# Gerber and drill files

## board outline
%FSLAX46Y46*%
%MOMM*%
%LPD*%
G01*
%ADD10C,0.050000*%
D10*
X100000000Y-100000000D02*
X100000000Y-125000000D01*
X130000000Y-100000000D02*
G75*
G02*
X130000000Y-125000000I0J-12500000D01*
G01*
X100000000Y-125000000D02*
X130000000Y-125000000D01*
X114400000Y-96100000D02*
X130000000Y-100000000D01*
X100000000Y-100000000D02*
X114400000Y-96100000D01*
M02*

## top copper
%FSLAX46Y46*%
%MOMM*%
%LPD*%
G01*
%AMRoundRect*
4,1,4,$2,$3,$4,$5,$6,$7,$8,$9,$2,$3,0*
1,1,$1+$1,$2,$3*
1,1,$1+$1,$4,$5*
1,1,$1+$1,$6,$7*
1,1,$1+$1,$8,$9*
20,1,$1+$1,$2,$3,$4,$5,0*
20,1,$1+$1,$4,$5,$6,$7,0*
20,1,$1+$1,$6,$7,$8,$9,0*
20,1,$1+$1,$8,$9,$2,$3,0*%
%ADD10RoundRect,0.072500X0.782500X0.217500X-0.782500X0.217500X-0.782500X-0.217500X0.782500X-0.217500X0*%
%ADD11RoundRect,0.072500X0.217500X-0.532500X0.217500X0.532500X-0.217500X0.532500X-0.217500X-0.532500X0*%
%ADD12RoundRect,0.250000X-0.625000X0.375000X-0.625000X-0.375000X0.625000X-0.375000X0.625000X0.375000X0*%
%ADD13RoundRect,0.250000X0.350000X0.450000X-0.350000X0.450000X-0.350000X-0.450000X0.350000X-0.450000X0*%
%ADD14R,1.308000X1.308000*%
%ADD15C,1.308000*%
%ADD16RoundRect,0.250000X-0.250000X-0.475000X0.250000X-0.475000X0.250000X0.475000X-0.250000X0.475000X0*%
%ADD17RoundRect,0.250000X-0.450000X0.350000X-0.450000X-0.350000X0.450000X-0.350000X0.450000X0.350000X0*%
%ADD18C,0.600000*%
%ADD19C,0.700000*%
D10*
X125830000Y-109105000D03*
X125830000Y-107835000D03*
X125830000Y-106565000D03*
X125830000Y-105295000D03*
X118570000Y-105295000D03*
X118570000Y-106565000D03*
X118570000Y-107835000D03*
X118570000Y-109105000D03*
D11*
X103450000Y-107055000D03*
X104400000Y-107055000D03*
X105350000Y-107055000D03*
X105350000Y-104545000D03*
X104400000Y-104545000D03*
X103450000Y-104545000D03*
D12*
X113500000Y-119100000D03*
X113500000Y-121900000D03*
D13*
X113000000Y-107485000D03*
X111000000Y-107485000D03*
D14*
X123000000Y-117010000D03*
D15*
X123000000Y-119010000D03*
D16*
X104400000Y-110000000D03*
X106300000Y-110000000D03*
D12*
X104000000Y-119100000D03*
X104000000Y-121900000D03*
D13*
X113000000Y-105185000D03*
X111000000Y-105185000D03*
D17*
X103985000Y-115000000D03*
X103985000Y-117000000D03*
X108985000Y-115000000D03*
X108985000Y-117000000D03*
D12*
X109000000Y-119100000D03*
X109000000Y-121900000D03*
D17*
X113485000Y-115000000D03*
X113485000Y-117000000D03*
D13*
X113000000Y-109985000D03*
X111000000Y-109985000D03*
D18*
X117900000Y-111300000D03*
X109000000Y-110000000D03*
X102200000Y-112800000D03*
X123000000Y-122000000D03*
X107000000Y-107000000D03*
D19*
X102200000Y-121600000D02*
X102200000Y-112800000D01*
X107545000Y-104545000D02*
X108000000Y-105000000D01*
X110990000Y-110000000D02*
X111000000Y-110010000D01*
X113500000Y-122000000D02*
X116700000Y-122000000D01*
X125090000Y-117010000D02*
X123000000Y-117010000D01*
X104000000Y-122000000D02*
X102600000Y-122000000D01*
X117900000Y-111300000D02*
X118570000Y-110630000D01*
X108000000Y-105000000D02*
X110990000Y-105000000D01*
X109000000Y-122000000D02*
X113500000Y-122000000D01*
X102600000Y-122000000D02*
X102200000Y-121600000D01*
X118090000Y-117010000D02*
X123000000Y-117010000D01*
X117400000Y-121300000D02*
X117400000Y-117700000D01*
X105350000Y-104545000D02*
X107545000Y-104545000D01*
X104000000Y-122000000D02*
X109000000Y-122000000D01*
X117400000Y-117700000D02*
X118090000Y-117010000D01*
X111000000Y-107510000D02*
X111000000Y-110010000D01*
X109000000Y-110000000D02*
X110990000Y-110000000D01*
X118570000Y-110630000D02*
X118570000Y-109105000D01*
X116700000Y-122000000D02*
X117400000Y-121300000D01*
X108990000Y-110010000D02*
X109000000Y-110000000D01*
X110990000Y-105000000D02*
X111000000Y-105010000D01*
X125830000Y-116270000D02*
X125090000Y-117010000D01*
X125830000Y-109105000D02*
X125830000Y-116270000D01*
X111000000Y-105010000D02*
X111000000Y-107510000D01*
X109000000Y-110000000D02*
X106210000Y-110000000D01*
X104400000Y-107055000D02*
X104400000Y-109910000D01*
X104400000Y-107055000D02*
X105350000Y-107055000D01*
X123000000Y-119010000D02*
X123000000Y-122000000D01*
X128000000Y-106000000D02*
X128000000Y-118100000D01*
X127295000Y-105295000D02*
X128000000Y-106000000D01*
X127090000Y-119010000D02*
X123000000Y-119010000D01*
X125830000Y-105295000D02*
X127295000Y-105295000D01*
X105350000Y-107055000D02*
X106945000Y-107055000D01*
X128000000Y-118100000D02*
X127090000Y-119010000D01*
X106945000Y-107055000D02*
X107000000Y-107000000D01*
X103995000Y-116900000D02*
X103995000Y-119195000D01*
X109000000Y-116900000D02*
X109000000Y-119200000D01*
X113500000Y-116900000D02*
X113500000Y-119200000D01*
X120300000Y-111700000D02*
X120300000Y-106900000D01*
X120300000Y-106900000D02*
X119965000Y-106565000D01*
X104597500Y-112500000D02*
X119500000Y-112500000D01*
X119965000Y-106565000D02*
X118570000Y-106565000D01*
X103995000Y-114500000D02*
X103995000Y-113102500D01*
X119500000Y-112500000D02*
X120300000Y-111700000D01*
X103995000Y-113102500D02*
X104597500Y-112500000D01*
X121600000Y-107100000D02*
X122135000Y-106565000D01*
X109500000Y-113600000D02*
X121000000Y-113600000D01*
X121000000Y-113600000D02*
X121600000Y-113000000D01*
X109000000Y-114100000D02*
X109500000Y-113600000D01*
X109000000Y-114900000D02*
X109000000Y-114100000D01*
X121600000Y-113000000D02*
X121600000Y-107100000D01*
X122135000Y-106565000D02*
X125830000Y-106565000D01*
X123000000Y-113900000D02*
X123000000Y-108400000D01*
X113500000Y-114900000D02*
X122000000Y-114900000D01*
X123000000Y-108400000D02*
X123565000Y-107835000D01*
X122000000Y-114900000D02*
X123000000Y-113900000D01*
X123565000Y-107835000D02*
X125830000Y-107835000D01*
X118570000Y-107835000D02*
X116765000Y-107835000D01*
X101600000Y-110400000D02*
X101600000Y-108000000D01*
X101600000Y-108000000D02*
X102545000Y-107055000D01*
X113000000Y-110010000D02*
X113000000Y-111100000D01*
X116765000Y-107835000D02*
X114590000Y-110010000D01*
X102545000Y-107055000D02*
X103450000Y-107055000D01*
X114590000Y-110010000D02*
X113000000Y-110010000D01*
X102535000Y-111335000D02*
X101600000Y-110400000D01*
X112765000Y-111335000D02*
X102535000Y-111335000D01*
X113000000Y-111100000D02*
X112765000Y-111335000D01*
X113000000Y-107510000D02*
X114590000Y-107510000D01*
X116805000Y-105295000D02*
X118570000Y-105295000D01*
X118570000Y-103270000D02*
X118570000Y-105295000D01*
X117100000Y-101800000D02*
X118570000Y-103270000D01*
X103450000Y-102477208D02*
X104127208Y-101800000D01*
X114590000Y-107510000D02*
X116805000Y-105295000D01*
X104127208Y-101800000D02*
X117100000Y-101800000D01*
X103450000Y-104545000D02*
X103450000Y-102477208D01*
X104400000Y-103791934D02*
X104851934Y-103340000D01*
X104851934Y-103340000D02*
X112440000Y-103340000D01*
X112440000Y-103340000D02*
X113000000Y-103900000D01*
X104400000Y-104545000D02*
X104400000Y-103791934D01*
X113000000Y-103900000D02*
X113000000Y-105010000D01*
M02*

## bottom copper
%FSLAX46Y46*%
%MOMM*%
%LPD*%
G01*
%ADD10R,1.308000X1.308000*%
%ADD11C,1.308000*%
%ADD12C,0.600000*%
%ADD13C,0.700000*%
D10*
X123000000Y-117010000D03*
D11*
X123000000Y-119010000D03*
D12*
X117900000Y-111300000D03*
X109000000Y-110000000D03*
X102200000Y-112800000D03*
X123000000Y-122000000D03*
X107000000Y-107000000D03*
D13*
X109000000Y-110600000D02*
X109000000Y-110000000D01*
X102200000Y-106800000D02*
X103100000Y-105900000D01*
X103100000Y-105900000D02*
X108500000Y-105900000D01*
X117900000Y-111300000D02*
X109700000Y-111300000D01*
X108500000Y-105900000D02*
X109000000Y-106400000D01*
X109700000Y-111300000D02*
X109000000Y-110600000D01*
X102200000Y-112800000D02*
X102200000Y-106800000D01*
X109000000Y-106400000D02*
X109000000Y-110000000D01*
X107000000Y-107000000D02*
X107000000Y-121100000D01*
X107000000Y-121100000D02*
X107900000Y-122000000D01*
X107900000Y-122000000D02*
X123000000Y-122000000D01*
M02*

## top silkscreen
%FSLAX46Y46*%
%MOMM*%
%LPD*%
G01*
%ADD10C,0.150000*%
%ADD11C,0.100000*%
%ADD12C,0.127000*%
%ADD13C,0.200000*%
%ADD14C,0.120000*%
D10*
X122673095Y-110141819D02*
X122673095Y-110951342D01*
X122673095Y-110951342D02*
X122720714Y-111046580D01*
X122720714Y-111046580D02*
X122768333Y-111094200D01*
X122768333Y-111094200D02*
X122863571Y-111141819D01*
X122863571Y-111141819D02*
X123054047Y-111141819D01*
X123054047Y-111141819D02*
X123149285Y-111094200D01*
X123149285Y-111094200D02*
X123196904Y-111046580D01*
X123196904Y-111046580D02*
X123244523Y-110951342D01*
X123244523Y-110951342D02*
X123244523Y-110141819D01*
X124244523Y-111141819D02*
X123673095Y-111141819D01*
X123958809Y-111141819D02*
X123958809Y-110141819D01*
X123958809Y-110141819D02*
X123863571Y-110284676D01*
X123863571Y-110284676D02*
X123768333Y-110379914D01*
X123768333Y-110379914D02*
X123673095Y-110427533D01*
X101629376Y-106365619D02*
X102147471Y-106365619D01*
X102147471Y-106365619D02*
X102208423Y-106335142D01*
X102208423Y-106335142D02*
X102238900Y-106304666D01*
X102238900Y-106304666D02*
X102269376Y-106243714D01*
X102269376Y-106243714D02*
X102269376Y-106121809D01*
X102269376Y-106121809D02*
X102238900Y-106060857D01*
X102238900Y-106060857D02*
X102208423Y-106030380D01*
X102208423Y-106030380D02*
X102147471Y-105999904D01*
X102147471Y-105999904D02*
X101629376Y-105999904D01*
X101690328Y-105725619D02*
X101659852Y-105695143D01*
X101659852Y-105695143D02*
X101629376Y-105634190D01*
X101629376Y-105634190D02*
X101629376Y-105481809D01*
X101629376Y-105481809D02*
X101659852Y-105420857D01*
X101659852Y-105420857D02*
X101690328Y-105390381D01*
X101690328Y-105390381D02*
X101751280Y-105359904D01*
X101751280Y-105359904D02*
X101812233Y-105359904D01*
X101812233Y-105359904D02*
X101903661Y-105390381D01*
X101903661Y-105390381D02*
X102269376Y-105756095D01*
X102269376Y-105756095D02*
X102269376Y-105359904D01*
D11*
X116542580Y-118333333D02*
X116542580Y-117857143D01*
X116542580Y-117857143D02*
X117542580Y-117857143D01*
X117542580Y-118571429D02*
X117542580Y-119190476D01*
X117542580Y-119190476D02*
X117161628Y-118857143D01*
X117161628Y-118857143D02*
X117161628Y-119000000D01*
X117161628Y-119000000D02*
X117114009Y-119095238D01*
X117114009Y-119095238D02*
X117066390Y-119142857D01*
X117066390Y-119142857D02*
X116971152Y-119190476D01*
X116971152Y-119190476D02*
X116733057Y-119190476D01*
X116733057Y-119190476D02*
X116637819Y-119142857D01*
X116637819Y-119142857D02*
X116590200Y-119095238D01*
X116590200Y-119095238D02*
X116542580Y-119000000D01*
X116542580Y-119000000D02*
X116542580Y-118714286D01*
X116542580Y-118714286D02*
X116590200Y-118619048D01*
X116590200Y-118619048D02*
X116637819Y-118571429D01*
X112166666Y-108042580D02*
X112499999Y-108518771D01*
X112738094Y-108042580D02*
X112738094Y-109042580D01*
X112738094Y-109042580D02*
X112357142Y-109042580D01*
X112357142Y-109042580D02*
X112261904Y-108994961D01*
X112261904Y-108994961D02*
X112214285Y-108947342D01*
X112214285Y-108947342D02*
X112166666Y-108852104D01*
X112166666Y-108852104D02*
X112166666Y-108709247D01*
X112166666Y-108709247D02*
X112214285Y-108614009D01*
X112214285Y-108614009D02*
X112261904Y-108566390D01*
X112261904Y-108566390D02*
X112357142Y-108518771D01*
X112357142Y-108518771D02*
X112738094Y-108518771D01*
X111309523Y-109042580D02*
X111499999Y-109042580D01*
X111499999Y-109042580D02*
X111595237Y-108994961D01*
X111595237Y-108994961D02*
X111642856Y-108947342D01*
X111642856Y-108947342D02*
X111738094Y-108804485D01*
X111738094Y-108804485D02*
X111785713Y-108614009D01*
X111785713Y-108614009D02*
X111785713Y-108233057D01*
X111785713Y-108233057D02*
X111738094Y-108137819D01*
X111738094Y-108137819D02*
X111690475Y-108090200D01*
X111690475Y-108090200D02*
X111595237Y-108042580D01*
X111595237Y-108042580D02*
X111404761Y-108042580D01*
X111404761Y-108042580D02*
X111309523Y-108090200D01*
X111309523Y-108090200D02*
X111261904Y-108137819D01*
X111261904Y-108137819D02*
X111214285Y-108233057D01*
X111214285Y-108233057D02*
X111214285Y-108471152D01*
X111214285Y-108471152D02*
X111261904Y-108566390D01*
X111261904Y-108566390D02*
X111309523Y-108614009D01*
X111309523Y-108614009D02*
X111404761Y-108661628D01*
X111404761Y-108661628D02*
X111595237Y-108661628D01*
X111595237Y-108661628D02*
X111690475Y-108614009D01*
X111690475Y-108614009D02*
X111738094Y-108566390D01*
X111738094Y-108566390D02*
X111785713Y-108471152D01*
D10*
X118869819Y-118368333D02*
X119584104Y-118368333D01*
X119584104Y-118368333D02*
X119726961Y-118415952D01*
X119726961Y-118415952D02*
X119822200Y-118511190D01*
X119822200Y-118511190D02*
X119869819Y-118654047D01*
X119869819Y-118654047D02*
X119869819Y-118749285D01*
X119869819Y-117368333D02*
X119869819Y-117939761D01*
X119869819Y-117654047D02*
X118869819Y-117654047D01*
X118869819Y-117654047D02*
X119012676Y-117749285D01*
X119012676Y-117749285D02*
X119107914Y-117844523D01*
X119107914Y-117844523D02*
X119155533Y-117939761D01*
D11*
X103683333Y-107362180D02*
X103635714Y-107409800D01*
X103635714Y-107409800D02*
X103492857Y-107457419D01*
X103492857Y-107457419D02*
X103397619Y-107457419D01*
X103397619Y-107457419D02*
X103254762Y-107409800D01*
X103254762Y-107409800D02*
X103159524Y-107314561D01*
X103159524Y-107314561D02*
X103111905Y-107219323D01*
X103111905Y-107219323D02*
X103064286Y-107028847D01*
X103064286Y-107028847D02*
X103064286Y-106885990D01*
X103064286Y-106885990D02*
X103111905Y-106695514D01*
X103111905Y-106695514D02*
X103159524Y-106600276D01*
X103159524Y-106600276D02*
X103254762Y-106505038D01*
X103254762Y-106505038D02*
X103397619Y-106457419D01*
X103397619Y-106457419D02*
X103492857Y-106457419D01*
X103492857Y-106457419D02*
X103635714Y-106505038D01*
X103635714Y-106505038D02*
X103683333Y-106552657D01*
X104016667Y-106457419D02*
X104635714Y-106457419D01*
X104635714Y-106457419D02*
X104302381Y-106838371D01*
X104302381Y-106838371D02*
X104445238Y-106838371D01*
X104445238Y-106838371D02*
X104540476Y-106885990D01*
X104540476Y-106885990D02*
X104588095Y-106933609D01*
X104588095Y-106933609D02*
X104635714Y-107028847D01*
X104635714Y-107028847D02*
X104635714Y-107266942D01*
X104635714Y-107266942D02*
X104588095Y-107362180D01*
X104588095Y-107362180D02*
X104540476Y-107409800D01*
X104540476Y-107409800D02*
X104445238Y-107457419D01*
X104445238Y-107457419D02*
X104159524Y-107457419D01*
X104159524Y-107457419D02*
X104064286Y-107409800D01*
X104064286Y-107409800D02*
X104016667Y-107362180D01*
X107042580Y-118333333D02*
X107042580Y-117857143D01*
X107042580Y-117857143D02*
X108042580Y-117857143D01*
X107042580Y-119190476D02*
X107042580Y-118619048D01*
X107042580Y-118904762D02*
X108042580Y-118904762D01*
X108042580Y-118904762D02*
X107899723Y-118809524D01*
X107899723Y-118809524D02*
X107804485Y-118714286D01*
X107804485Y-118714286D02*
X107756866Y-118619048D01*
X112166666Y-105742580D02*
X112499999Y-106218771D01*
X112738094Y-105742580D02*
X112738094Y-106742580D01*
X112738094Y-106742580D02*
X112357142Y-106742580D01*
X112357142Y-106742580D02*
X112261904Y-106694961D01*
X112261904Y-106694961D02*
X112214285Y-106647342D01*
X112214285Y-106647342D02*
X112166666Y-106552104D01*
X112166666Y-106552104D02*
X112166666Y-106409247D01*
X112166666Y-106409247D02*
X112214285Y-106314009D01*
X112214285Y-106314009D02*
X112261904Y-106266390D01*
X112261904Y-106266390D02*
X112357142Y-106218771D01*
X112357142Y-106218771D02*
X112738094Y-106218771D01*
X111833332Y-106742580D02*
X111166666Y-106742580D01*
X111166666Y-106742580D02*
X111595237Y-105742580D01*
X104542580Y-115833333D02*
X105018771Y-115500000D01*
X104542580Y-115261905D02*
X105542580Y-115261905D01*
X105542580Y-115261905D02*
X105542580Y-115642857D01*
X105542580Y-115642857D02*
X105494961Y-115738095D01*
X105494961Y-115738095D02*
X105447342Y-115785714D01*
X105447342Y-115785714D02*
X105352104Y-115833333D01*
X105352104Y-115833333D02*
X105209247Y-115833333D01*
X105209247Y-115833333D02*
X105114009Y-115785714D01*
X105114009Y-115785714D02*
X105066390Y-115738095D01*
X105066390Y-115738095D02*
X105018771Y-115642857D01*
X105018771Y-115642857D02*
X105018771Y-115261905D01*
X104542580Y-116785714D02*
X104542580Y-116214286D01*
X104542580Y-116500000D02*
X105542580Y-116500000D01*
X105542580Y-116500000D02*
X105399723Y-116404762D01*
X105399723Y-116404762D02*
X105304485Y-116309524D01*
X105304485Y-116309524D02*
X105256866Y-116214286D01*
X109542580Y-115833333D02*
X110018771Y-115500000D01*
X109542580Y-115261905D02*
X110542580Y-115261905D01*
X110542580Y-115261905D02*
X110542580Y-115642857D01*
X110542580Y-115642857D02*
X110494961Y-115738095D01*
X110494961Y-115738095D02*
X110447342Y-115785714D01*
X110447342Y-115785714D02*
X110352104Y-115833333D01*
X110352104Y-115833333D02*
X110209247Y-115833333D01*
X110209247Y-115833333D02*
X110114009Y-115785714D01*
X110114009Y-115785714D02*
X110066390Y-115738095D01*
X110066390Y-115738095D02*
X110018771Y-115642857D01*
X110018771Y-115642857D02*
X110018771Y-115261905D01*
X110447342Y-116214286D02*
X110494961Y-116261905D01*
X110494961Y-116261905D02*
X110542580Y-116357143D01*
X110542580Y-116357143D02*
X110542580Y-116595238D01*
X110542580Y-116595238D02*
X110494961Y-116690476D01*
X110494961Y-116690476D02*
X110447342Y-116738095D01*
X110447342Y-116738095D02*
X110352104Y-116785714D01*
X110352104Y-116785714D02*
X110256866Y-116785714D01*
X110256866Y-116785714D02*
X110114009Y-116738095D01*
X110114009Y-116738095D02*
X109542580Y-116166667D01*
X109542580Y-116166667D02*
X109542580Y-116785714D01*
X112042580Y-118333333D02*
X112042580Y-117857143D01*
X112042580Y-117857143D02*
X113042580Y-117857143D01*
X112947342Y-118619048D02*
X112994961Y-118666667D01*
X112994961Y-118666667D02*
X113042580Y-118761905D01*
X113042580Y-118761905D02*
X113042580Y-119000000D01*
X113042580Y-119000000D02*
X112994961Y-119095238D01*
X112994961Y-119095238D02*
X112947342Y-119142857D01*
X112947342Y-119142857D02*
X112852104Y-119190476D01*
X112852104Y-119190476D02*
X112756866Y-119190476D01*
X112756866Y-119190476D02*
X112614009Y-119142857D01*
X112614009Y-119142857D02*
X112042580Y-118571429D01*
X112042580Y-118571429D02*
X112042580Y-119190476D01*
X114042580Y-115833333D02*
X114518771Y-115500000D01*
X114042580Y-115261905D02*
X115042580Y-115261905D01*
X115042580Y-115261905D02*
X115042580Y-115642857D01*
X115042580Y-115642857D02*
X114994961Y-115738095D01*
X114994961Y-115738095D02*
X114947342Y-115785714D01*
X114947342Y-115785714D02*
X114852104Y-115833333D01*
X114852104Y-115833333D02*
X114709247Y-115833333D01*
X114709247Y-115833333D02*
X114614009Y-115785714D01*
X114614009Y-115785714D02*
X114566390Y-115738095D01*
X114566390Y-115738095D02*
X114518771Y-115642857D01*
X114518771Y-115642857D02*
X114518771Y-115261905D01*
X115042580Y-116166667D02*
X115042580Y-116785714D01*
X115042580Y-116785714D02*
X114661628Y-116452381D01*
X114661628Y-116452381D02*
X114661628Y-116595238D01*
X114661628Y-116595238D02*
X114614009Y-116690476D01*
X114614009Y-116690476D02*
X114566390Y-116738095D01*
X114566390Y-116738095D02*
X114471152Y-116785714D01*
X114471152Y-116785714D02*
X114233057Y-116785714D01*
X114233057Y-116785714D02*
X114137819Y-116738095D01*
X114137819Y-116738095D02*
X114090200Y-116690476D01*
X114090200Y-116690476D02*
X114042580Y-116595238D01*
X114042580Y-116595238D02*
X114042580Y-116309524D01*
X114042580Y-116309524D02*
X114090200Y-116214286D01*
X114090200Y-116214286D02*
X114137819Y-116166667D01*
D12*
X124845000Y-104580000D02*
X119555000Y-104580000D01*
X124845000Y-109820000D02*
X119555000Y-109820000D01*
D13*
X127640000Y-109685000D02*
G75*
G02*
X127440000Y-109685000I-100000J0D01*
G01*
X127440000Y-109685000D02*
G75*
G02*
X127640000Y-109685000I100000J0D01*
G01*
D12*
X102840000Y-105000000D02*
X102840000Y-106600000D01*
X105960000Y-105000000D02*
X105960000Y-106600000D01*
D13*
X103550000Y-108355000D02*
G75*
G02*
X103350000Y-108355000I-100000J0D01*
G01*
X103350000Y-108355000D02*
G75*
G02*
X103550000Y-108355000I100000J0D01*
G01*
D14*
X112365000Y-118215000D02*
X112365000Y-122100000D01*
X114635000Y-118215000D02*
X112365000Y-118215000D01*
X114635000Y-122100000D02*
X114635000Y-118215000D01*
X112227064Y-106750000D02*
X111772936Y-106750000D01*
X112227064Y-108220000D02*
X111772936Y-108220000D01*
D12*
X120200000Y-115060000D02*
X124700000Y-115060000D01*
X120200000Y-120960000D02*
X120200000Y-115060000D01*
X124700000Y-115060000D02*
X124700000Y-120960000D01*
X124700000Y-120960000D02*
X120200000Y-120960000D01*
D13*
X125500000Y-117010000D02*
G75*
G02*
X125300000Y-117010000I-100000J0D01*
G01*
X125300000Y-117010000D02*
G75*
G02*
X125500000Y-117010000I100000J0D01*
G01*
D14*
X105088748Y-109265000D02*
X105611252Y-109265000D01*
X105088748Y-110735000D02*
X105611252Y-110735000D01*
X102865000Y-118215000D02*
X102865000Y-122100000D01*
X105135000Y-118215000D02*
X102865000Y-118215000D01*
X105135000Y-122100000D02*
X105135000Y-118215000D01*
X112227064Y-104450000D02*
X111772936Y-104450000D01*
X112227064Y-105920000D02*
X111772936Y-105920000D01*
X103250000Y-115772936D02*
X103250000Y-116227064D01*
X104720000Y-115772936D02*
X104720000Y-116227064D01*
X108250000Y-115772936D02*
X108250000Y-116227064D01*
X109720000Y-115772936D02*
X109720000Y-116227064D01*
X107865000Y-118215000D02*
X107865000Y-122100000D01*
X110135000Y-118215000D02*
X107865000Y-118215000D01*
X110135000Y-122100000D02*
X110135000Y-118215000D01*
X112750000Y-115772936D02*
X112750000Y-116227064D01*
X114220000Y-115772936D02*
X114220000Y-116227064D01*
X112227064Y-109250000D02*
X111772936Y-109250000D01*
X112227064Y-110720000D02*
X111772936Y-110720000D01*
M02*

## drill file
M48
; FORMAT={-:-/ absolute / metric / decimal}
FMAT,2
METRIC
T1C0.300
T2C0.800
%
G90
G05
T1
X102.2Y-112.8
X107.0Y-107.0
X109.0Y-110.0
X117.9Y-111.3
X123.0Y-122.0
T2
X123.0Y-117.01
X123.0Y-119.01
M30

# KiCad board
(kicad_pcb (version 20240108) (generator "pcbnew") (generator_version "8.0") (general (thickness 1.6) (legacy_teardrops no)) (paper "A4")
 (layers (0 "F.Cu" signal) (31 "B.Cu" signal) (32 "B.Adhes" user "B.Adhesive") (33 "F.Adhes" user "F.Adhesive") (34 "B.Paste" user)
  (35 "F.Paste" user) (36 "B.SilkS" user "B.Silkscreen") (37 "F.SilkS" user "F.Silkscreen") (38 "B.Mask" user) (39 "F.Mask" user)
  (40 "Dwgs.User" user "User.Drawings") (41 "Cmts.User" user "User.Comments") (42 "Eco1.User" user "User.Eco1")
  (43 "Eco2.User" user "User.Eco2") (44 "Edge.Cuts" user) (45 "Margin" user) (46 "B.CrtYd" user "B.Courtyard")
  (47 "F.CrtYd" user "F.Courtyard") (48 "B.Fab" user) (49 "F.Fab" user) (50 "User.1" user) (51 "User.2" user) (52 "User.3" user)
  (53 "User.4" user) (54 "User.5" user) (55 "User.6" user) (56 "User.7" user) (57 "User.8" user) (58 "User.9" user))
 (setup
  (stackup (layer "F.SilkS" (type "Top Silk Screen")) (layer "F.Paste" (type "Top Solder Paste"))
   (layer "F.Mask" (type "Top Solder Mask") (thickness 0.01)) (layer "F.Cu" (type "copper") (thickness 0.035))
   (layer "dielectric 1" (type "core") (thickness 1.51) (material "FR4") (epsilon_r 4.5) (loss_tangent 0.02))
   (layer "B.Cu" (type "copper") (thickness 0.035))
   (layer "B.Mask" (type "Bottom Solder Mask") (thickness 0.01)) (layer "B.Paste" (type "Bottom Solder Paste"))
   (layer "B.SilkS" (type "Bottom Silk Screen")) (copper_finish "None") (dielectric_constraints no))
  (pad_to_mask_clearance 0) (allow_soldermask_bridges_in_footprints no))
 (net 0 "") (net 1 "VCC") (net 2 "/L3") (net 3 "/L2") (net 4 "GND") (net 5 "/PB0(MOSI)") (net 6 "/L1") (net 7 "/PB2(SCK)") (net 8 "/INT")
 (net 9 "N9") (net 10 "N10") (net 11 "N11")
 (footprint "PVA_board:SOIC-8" (layer "F.Cu") (at 122.2 107.2 180)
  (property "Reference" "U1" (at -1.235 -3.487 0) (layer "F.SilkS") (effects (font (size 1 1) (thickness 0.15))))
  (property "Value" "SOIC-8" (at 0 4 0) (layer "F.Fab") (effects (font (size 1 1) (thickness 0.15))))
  (fp_line (start -2.645 2.62) (end 2.645 2.62) (stroke (width 0.127) (type solid)) (layer "F.SilkS"))
  (fp_line (start -2.645 -2.62) (end 2.645 -2.62) (stroke (width 0.127) (type solid)) (layer "F.SilkS"))
  (fp_circle (center -5.34 -2.485) (end -5.24 -2.485) (stroke (width 0.2) (type solid)) (fill none) (layer "F.SilkS"))
  (pad "1" smd roundrect (at -3.63 -1.905 180) (size 1.71 0.58) (layers "F.Cu" "F.Paste" "F.Mask") (roundrect_rratio 0.125) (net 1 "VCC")
   (solder_mask_margin 0.102))
  (pad "2" smd roundrect (at -3.63 -0.635 180) (size 1.71 0.58) (layers "F.Cu" "F.Paste" "F.Mask") (roundrect_rratio 0.125) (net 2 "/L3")
   (solder_mask_margin 0.102))
  (pad "3" smd roundrect (at -3.63 0.635 180) (size 1.71 0.58) (layers "F.Cu" "F.Paste" "F.Mask") (roundrect_rratio 0.125) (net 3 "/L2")
   (solder_mask_margin 0.102))
  (pad "4" smd roundrect (at -3.63 1.905 180) (size 1.71 0.58) (layers "F.Cu" "F.Paste" "F.Mask") (roundrect_rratio 0.125) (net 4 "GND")
   (solder_mask_margin 0.102))
  (pad "5" smd roundrect (at 3.63 1.905 180) (size 1.71 0.58) (layers "F.Cu" "F.Paste" "F.Mask") (roundrect_rratio 0.125)
   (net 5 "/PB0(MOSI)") (solder_mask_margin 0.102))
  (pad "6" smd roundrect (at 3.63 0.635 180) (size 1.71 0.58) (layers "F.Cu" "F.Paste" "F.Mask") (roundrect_rratio 0.125) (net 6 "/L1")
   (solder_mask_margin 0.102))
  (pad "7" smd roundrect (at 3.63 -0.635 180) (size 1.71 0.58) (layers "F.Cu" "F.Paste" "F.Mask") (roundrect_rratio 0.125)
   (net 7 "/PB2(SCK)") (solder_mask_margin 0.102))
  (pad "8" smd roundrect (at 3.63 -1.905 180) (size 1.71 0.58) (layers "F.Cu" "F.Paste" "F.Mask") (roundrect_rratio 0.125) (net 1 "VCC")
   (solder_mask_margin 0.102)))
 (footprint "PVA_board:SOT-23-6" (layer "F.Cu") (at 104.4 105.8 90)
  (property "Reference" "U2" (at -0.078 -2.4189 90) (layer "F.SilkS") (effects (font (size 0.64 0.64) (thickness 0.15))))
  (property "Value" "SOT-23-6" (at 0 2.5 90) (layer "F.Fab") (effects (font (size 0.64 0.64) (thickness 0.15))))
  (fp_line (start 0.8 -1.56) (end -0.8 -1.56) (stroke (width 0.127) (type solid)) (layer "F.SilkS"))
  (fp_line (start 0.8 1.56) (end -0.8 1.56) (stroke (width 0.127) (type solid)) (layer "F.SilkS"))
  (fp_circle (center -2.555 -0.95) (end -2.455 -0.95) (stroke (width 0.2) (type solid)) (fill none) (layer "F.SilkS"))
  (pad "1" smd roundrect (at -1.255 -0.95 90) (size 1.21 0.58) (layers "F.Cu" "F.Paste" "F.Mask") (roundrect_rratio 0.125)
   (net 7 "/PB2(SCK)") (solder_mask_margin 0.102))
  (pad "2" smd roundrect (at -1.255 0 90) (size 1.21 0.58) (layers "F.Cu" "F.Paste" "F.Mask") (roundrect_rratio 0.125) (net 4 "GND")
   (solder_mask_margin 0.102))
  (pad "3" smd roundrect (at -1.255 0.95 90) (size 1.21 0.58) (layers "F.Cu" "F.Paste" "F.Mask") (roundrect_rratio 0.125) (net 4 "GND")
   (solder_mask_margin 0.102))
  (pad "4" smd roundrect (at 1.255 0.95 90) (size 1.21 0.58) (layers "F.Cu" "F.Paste" "F.Mask") (roundrect_rratio 0.125) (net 1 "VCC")
   (solder_mask_margin 0.102))
  (pad "5" smd roundrect (at 1.255 0 90) (size 1.21 0.58) (layers "F.Cu" "F.Paste" "F.Mask") (roundrect_rratio 0.125) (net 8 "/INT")
   (solder_mask_margin 0.102))
  (pad "6" smd roundrect (at 1.255 -0.95 90) (size 1.21 0.58) (layers "F.Cu" "F.Paste" "F.Mask") (roundrect_rratio 0.125)
   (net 5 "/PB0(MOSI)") (solder_mask_margin 0.102)))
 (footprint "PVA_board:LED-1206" (layer "F.Cu") (at 113.5 120.5 -90)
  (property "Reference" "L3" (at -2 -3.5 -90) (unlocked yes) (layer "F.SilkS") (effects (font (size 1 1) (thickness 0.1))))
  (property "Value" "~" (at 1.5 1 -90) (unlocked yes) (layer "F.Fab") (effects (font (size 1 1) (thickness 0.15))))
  (fp_line (start -2.285 1.135) (end 1.6 1.135) (stroke (width 0.12) (type solid)) (layer "F.SilkS"))
  (fp_line (start -2.285 -1.135) (end -2.285 1.135) (stroke (width 0.12) (type solid)) (layer "F.SilkS"))
  (fp_line (start 1.6 -1.135) (end -2.285 -1.135) (stroke (width 0.12) (type solid)) (layer "F.SilkS"))
  (pad "1" smd roundrect (at -1.4 0 270) (size 1.25 1.75) (layers "F.Cu" "F.Paste" "F.Mask") (roundrect_rratio 0.2) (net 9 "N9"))
  (pad "2" smd roundrect (at 1.4 0 270) (size 1.25 1.75) (layers "F.Cu" "F.Paste" "F.Mask") (roundrect_rratio 0.2) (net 1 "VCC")))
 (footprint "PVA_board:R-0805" (layer "F.Cu") (at 112 107.5 180)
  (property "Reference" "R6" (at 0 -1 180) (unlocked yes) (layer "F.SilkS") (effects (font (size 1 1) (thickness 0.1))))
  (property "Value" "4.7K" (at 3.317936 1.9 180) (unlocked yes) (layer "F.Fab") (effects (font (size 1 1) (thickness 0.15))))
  (fp_line (start -0.227064 0.75) (end 0.227064 0.75) (stroke (width 0.12) (type solid)) (layer "F.SilkS"))
  (fp_line (start -0.227064 -0.72) (end 0.227064 -0.72) (stroke (width 0.12) (type solid)) (layer "F.SilkS"))
  (pad "1" smd roundrect (at -1 0.015 180) (size 1.2 1.4) (layers "F.Cu" "F.Paste" "F.Mask") (roundrect_rratio 0.208333)
   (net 5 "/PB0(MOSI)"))
  (pad "2" smd roundrect (at 1 0.015 180) (size 1.2 1.4) (layers "F.Cu" "F.Paste" "F.Mask") (roundrect_rratio 0.208333) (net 1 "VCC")))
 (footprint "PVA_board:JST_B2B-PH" (layer "F.Cu") (at 123 118.01 90)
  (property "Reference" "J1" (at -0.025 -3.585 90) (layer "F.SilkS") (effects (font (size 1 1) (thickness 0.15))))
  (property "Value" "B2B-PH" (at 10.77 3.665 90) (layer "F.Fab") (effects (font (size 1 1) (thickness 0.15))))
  (fp_line (start 2.95 -2.8) (end 2.95 1.7) (stroke (width 0.127) (type solid)) (layer "F.SilkS"))
  (fp_line (start -2.95 -2.8) (end 2.95 -2.8) (stroke (width 0.127) (type solid)) (layer "F.SilkS"))
  (fp_line (start 2.95 1.7) (end -2.95 1.7) (stroke (width 0.127) (type solid)) (layer "F.SilkS"))
  (fp_line (start -2.95 1.7) (end -2.95 -2.8) (stroke (width 0.127) (type solid)) (layer "F.SilkS"))
  (fp_circle (center 1 2.4) (end 1.1 2.4) (stroke (width 0.2) (type solid)) (fill none) (layer "F.SilkS"))
  (pad "1" thru_hole rect (at 1 0 90) (size 1.308 1.308) (drill 0.8) (layers "*.Cu" "*.Mask") (remove_unused_layers no) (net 1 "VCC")
   (solder_mask_margin 0.102))
  (pad "2" thru_hole circle (at -1 0 90) (size 1.308 1.308) (drill 0.8) (layers "*.Cu" "*.Mask") (remove_unused_layers no) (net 4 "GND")
   (solder_mask_margin 0.102)))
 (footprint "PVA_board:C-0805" (layer "F.Cu") (at 105.35 110)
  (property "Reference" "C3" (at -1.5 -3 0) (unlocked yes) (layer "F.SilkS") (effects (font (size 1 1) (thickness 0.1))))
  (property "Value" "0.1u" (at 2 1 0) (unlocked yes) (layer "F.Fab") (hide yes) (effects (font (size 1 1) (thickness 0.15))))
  (fp_line (start -0.261252 -0.735) (end 0.261252 -0.735) (stroke (width 0.12) (type solid)) (layer "F.SilkS"))
  (fp_line (start -0.261252 0.735) (end 0.261252 0.735) (stroke (width 0.12) (type solid)) (layer "F.SilkS"))
  (pad "1" smd roundrect (at -0.95 0) (size 1 1.45) (layers "F.Cu" "F.Paste" "F.Mask") (roundrect_rratio 0.25) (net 4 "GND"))
  (pad "2" smd roundrect (at 0.95 0) (size 1 1.45) (layers "F.Cu" "F.Paste" "F.Mask") (roundrect_rratio 0.25) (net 1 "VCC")))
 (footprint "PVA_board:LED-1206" (layer "F.Cu") (at 104 120.5 -90)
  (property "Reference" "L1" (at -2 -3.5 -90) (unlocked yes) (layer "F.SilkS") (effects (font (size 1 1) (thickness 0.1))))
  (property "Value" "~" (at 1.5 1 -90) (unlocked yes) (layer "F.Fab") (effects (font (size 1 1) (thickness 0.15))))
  (fp_line (start -2.285 1.135) (end 1.6 1.135) (stroke (width 0.12) (type solid)) (layer "F.SilkS"))
  (fp_line (start -2.285 -1.135) (end -2.285 1.135) (stroke (width 0.12) (type solid)) (layer "F.SilkS"))
  (fp_line (start 1.6 -1.135) (end -2.285 -1.135) (stroke (width 0.12) (type solid)) (layer "F.SilkS"))
  (pad "1" smd roundrect (at -1.4 0 270) (size 1.25 1.75) (layers "F.Cu" "F.Paste" "F.Mask") (roundrect_rratio 0.2) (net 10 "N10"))
  (pad "2" smd roundrect (at 1.4 0 270) (size 1.25 1.75) (layers "F.Cu" "F.Paste" "F.Mask") (roundrect_rratio 0.2) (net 1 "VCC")))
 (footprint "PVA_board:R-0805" (layer "F.Cu") (at 112 105.2 180)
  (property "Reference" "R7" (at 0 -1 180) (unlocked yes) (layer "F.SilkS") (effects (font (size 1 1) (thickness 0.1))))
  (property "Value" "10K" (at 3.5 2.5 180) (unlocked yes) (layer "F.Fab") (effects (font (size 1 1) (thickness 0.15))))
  (fp_line (start -0.227064 0.75) (end 0.227064 0.75) (stroke (width 0.12) (type solid)) (layer "F.SilkS"))
  (fp_line (start -0.227064 -0.72) (end 0.227064 -0.72) (stroke (width 0.12) (type solid)) (layer "F.SilkS"))
  (pad "1" smd roundrect (at -1 0.015 180) (size 1.2 1.4) (layers "F.Cu" "F.Paste" "F.Mask") (roundrect_rratio 0.208333) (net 8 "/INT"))
  (pad "2" smd roundrect (at 1 0.015 180) (size 1.2 1.4) (layers "F.Cu" "F.Paste" "F.Mask") (roundrect_rratio 0.208333) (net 1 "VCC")))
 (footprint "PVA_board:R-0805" (layer "F.Cu") (at 104 116 -90)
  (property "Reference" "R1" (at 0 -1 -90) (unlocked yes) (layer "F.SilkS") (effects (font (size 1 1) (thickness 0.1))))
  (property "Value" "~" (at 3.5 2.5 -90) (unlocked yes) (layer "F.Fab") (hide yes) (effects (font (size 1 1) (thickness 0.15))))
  (fp_line (start -0.227064 0.75) (end 0.227064 0.75) (stroke (width 0.12) (type solid)) (layer "F.SilkS"))
  (fp_line (start -0.227064 -0.72) (end 0.227064 -0.72) (stroke (width 0.12) (type solid)) (layer "F.SilkS"))
  (pad "1" smd roundrect (at -1 0.015 270) (size 1.2 1.4) (layers "F.Cu" "F.Paste" "F.Mask") (roundrect_rratio 0.208333) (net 6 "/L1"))
  (pad "2" smd roundrect (at 1 0.015 270) (size 1.2 1.4) (layers "F.Cu" "F.Paste" "F.Mask") (roundrect_rratio 0.208333) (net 10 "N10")))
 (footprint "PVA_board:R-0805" (layer "F.Cu") (at 109 116 -90)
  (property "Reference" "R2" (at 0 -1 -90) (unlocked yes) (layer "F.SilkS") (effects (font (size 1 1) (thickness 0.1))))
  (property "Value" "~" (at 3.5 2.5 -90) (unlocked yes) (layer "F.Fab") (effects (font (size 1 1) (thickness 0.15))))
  (fp_line (start -0.227064 0.75) (end 0.227064 0.75) (stroke (width 0.12) (type solid)) (layer "F.SilkS"))
  (fp_line (start -0.227064 -0.72) (end 0.227064 -0.72) (stroke (width 0.12) (type solid)) (layer "F.SilkS"))
  (pad "1" smd roundrect (at -1 0.015 270) (size 1.2 1.4) (layers "F.Cu" "F.Paste" "F.Mask") (roundrect_rratio 0.208333) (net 3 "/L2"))
  (pad "2" smd roundrect (at 1 0.015 270) (size 1.2 1.4) (layers "F.Cu" "F.Paste" "F.Mask") (roundrect_rratio 0.208333) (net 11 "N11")))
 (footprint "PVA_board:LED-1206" (layer "F.Cu") (at 109 120.5 -90)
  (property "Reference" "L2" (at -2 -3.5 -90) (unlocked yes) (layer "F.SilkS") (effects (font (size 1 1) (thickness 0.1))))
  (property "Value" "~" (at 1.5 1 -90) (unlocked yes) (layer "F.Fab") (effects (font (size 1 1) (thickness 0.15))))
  (fp_line (start -2.285 1.135) (end 1.6 1.135) (stroke (width 0.12) (type solid)) (layer "F.SilkS"))
  (fp_line (start -2.285 -1.135) (end -2.285 1.135) (stroke (width 0.12) (type solid)) (layer "F.SilkS"))
  (fp_line (start 1.6 -1.135) (end -2.285 -1.135) (stroke (width 0.12) (type solid)) (layer "F.SilkS"))
  (pad "1" smd roundrect (at -1.4 0 270) (size 1.25 1.75) (layers "F.Cu" "F.Paste" "F.Mask") (roundrect_rratio 0.2) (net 11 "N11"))
  (pad "2" smd roundrect (at 1.4 0 270) (size 1.25 1.75) (layers "F.Cu" "F.Paste" "F.Mask") (roundrect_rratio 0.2) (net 1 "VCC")))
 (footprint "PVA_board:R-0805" (layer "F.Cu") (at 113.5 116 -90)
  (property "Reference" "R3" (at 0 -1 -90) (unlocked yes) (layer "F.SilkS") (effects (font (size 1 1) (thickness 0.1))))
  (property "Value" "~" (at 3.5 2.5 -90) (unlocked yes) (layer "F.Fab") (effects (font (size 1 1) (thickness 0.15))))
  (fp_line (start -0.227064 0.75) (end 0.227064 0.75) (stroke (width 0.12) (type solid)) (layer "F.SilkS"))
  (fp_line (start -0.227064 -0.72) (end 0.227064 -0.72) (stroke (width 0.12) (type solid)) (layer "F.SilkS"))
  (pad "1" smd roundrect (at -1 0.015 270) (size 1.2 1.4) (layers "F.Cu" "F.Paste" "F.Mask") (roundrect_rratio 0.208333) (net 2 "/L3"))
  (pad "2" smd roundrect (at 1 0.015 270) (size 1.2 1.4) (layers "F.Cu" "F.Paste" "F.Mask") (roundrect_rratio 0.208333) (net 9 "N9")))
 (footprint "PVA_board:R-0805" (layer "F.Cu") (at 112 110 180)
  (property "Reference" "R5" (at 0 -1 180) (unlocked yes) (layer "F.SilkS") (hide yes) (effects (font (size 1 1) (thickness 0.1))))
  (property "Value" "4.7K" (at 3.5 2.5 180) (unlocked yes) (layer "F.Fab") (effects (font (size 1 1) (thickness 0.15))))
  (fp_line (start -0.227064 0.75) (end 0.227064 0.75) (stroke (width 0.12) (type solid)) (layer "F.SilkS"))
  (fp_line (start -0.227064 -0.72) (end 0.227064 -0.72) (stroke (width 0.12) (type solid)) (layer "F.SilkS"))
  (pad "1" smd roundrect (at -1 0.015 180) (size 1.2 1.4) (layers "F.Cu" "F.Paste" "F.Mask") (roundrect_rratio 0.208333) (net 7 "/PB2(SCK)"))
  (pad "2" smd roundrect (at 1 0.015 180) (size 1.2 1.4) (layers "F.Cu" "F.Paste" "F.Mask") (roundrect_rratio 0.208333) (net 1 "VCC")))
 (gr_line (start 100 100) (end 100 125) (stroke (width 0.05) (type default)) (layer "Edge.Cuts"))
 (gr_arc (start 130 100) (mid 142.5 112.5) (end 130 125) (stroke (width 0.05) (type default)) (layer "Edge.Cuts"))
 (gr_line (start 100 125) (end 130 125) (stroke (width 0.05) (type default)) (layer "Edge.Cuts"))
 (gr_line (start 114.4 96.1) (end 130 100) (stroke (width 0.05) (type default)) (layer "Edge.Cuts"))
 (gr_line (start 100 100) (end 114.4 96.1) (stroke (width 0.05) (type default)) (layer "Edge.Cuts"))
 (segment (start 102.2 121.6) (end 102.2 112.8) (width 0.7) (layer "F.Cu") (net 1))
 (segment (start 107.545 104.545) (end 108 105) (width 0.7) (layer "F.Cu") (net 1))
 (segment (start 110.99 110) (end 111 110.01) (width 0.7) (layer "F.Cu") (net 1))
 (segment (start 113.5 122) (end 116.7 122) (width 0.7) (layer "F.Cu") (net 1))
 (segment (start 125.09 117.01) (end 123 117.01) (width 0.7) (layer "F.Cu") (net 1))
 (segment (start 104 122) (end 102.6 122) (width 0.7) (layer "F.Cu") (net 1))
 (segment (start 117.9 111.3) (end 118.57 110.63) (width 0.7) (layer "F.Cu") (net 1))
 (segment (start 108 105) (end 110.99 105) (width 0.7) (layer "F.Cu") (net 1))
 (segment (start 109 122) (end 113.5 122) (width 0.7) (layer "F.Cu") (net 1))
 (segment (start 102.6 122) (end 102.2 121.6) (width 0.7) (layer "F.Cu") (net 1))
 (segment (start 118.09 117.01) (end 123 117.01) (width 0.7) (layer "F.Cu") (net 1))
 (segment (start 117.4 121.3) (end 117.4 117.7) (width 0.7) (layer "F.Cu") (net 1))
 (segment (start 105.35 104.545) (end 107.545 104.545) (width 0.7) (layer "F.Cu") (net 1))
 (segment (start 104 122) (end 109 122) (width 0.7) (layer "F.Cu") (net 1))
 (segment (start 117.4 117.7) (end 118.09 117.01) (width 0.7) (layer "F.Cu") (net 1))
 (segment (start 111 107.51) (end 111 110.01) (width 0.7) (layer "F.Cu") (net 1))
 (segment (start 109 110) (end 110.99 110) (width 0.7) (layer "F.Cu") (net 1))
 (segment (start 118.57 110.63) (end 118.57 109.105) (width 0.7) (layer "F.Cu") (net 1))
 (segment (start 116.7 122) (end 117.4 121.3) (width 0.7) (layer "F.Cu") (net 1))
 (segment (start 108.99 110.01) (end 109 110) (width 0.7) (layer "F.Cu") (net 1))
 (segment (start 110.99 105) (end 111 105.01) (width 0.7) (layer "F.Cu") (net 1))
 (segment (start 125.83 116.27) (end 125.09 117.01) (width 0.7) (layer "F.Cu") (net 1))
 (segment (start 125.83 109.105) (end 125.83 116.27) (width 0.7) (layer "F.Cu") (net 1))
 (segment (start 111 105.01) (end 111 107.51) (width 0.7) (layer "F.Cu") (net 1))
 (segment (start 109 110) (end 106.21 110) (width 0.7) (layer "F.Cu") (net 1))
 (via (at 117.9 111.3) (size 0.6) (drill 0.3) (layers "F.Cu" "B.Cu") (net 1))
 (via (at 109 110) (size 0.6) (drill 0.3) (layers "F.Cu" "B.Cu") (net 1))
 (via (at 102.2 112.8) (size 0.6) (drill 0.3) (layers "F.Cu" "B.Cu") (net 1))
 (segment (start 109 110.6) (end 109 110) (width 0.7) (layer "B.Cu") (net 1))
 (segment (start 102.2 106.8) (end 103.1 105.9) (width 0.7) (layer "B.Cu") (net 1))
 (segment (start 103.1 105.9) (end 108.5 105.9) (width 0.7) (layer "B.Cu") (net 1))
 (segment (start 117.9 111.3) (end 109.7 111.3) (width 0.7) (layer "B.Cu") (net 1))
 (segment (start 108.5 105.9) (end 109 106.4) (width 0.7) (layer "B.Cu") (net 1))
 (segment (start 109.7 111.3) (end 109 110.6) (width 0.7) (layer "B.Cu") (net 1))
 (segment (start 102.2 112.8) (end 102.2 106.8) (width 0.7) (layer "B.Cu") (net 1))
 (segment (start 109 106.4) (end 109 110) (width 0.7) (layer "B.Cu") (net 1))
 (segment (start 104.4 107.055) (end 104.4 109.91) (width 0.7) (layer "F.Cu") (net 4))
 (segment (start 104.4 107.055) (end 105.35 107.055) (width 0.7) (layer "F.Cu") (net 4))
 (segment (start 123 119.01) (end 123 122) (width 0.7) (layer "F.Cu") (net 4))
 (segment (start 128 106) (end 128 118.1) (width 0.7) (layer "F.Cu") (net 4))
 (segment (start 127.295 105.295) (end 128 106) (width 0.7) (layer "F.Cu") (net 4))
 (segment (start 127.09 119.01) (end 123 119.01) (width 0.7) (layer "F.Cu") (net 4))
 (segment (start 125.83 105.295) (end 127.295 105.295) (width 0.7) (layer "F.Cu") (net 4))
 (segment (start 105.35 107.055) (end 106.945 107.055) (width 0.7) (layer "F.Cu") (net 4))
 (segment (start 128 118.1) (end 127.09 119.01) (width 0.7) (layer "F.Cu") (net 4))
 (segment (start 106.945 107.055) (end 107 107) (width 0.7) (layer "F.Cu") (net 4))
 (via (at 123 122) (size 0.6) (drill 0.3) (layers "F.Cu" "B.Cu") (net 4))
 (via (at 107 107) (size 0.6) (drill 0.3) (layers "F.Cu" "B.Cu") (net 4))
 (segment (start 107 107) (end 107 121.1) (width 0.7) (layer "B.Cu") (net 4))
 (segment (start 107 121.1) (end 107.9 122) (width 0.7) (layer "B.Cu") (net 4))
 (segment (start 107.9 122) (end 123 122) (width 0.7) (layer "B.Cu") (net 4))
 (segment (start 103.995 116.9) (end 103.995 119.195) (width 0.7) (layer "F.Cu") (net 10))
 (segment (start 109 116.9) (end 109 119.2) (width 0.7) (layer "F.Cu") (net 11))
 (segment (start 113.5 116.9) (end 113.5 119.2) (width 0.7) (layer "F.Cu") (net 9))
 (segment (start 120.3 111.7) (end 120.3 106.9) (width 0.7) (layer "F.Cu") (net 6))
 (segment (start 120.3 106.9) (end 119.965 106.565) (width 0.7) (layer "F.Cu") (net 6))
 (segment (start 104.5975 112.5) (end 119.5 112.5) (width 0.7) (locked yes) (layer "F.Cu") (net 6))
 (segment (start 119.965 106.565) (end 118.57 106.565) (width 0.7) (layer "F.Cu") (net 6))
 (segment (start 103.995 114.5) (end 103.995 113.1025) (width 0.7) (layer "F.Cu") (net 6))
 (segment (start 119.5 112.5) (end 120.3 111.7) (width 0.7) (layer "F.Cu") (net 6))
 (segment (start 103.995 113.1025) (end 104.5975 112.5) (width 0.7) (layer "F.Cu") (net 6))
 (segment (start 121.6 107.1) (end 122.135 106.565) (width 0.7) (layer "F.Cu") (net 3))
 (segment (start 109.5 113.6) (end 121 113.6) (width 0.7) (layer "F.Cu") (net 3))
 (segment (start 121 113.6) (end 121.6 113) (width 0.7) (layer "F.Cu") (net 3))
 (segment (start 109 114.1) (end 109.5 113.6) (width 0.7) (layer "F.Cu") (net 3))
 (segment (start 109 114.9) (end 109 114.1) (width 0.7) (layer "F.Cu") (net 3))
 (segment (start 121.6 113) (end 121.6 107.1) (width 0.7) (layer "F.Cu") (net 3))
 (segment (start 122.135 106.565) (end 125.83 106.565) (width 0.7) (layer "F.Cu") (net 3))
 (segment (start 123 113.9) (end 123 108.4) (width 0.7) (layer "F.Cu") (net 2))
 (segment (start 113.5 114.9) (end 122 114.9) (width 0.7) (layer "F.Cu") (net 2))
 (segment (start 123 108.4) (end 123.565 107.835) (width 0.7) (layer "F.Cu") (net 2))
 (segment (start 122 114.9) (end 123 113.9) (width 0.7) (layer "F.Cu") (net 2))
 (segment (start 123.565 107.835) (end 125.83 107.835) (width 0.7) (layer "F.Cu") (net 2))
 (segment (start 118.57 107.835) (end 116.765 107.835) (width 0.7) (layer "F.Cu") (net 7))
 (segment (start 101.6 110.4) (end 101.6 108) (width 0.7) (layer "F.Cu") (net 7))
 (segment (start 101.6 108) (end 102.545 107.055) (width 0.7) (layer "F.Cu") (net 7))
 (segment (start 113 110.01) (end 113 111.1) (width 0.7) (layer "F.Cu") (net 7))
 (segment (start 116.765 107.835) (end 114.59 110.01) (width 0.7) (layer "F.Cu") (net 7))
 (segment (start 102.545 107.055) (end 103.45 107.055) (width 0.7) (layer "F.Cu") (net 7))
 (segment (start 114.59 110.01) (end 113 110.01) (width 0.7) (layer "F.Cu") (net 7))
 (segment (start 102.535 111.335) (end 101.6 110.4) (width 0.7) (layer "F.Cu") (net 7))
 (segment (start 112.765 111.335) (end 102.535 111.335) (width 0.7) (layer "F.Cu") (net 7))
 (segment (start 113 111.1) (end 112.765 111.335) (width 0.7) (layer "F.Cu") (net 7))
 (segment (start 113 107.51) (end 114.59 107.51) (width 0.7) (layer "F.Cu") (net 5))
 (segment (start 116.805 105.295) (end 118.57 105.295) (width 0.7) (layer "F.Cu") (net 5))
 (segment (start 118.57 103.27) (end 118.57 105.295) (width 0.7) (layer "F.Cu") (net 5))
 (segment (start 117.1 101.8) (end 118.57 103.27) (width 0.7) (layer "F.Cu") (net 5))
 (segment (start 103.45 102.477208) (end 104.127208 101.8) (width 0.7) (layer "F.Cu") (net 5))
 (segment (start 114.59 107.51) (end 116.805 105.295) (width 0.7) (layer "F.Cu") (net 5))
 (segment (start 104.127208 101.8) (end 117.1 101.8) (width 0.7) (layer "F.Cu") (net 5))
 (segment (start 103.45 104.545) (end 103.45 102.477208) (width 0.7) (layer "F.Cu") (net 5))
 (segment (start 104.4 103.791934) (end 104.851934 103.34) (width 0.7) (layer "F.Cu") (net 8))
 (segment (start 104.851934 103.34) (end 112.44 103.34) (width 0.7) (layer "F.Cu") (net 8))
 (segment (start 112.44 103.34) (end 113 103.9) (width 0.7) (layer "F.Cu") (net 8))
 (segment (start 104.4 104.545) (end 104.4 103.791934) (width 0.7) (layer "F.Cu") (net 8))
 (segment (start 113 103.9) (end 113 105.01) (width 0.7) (layer "F.Cu") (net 8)))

